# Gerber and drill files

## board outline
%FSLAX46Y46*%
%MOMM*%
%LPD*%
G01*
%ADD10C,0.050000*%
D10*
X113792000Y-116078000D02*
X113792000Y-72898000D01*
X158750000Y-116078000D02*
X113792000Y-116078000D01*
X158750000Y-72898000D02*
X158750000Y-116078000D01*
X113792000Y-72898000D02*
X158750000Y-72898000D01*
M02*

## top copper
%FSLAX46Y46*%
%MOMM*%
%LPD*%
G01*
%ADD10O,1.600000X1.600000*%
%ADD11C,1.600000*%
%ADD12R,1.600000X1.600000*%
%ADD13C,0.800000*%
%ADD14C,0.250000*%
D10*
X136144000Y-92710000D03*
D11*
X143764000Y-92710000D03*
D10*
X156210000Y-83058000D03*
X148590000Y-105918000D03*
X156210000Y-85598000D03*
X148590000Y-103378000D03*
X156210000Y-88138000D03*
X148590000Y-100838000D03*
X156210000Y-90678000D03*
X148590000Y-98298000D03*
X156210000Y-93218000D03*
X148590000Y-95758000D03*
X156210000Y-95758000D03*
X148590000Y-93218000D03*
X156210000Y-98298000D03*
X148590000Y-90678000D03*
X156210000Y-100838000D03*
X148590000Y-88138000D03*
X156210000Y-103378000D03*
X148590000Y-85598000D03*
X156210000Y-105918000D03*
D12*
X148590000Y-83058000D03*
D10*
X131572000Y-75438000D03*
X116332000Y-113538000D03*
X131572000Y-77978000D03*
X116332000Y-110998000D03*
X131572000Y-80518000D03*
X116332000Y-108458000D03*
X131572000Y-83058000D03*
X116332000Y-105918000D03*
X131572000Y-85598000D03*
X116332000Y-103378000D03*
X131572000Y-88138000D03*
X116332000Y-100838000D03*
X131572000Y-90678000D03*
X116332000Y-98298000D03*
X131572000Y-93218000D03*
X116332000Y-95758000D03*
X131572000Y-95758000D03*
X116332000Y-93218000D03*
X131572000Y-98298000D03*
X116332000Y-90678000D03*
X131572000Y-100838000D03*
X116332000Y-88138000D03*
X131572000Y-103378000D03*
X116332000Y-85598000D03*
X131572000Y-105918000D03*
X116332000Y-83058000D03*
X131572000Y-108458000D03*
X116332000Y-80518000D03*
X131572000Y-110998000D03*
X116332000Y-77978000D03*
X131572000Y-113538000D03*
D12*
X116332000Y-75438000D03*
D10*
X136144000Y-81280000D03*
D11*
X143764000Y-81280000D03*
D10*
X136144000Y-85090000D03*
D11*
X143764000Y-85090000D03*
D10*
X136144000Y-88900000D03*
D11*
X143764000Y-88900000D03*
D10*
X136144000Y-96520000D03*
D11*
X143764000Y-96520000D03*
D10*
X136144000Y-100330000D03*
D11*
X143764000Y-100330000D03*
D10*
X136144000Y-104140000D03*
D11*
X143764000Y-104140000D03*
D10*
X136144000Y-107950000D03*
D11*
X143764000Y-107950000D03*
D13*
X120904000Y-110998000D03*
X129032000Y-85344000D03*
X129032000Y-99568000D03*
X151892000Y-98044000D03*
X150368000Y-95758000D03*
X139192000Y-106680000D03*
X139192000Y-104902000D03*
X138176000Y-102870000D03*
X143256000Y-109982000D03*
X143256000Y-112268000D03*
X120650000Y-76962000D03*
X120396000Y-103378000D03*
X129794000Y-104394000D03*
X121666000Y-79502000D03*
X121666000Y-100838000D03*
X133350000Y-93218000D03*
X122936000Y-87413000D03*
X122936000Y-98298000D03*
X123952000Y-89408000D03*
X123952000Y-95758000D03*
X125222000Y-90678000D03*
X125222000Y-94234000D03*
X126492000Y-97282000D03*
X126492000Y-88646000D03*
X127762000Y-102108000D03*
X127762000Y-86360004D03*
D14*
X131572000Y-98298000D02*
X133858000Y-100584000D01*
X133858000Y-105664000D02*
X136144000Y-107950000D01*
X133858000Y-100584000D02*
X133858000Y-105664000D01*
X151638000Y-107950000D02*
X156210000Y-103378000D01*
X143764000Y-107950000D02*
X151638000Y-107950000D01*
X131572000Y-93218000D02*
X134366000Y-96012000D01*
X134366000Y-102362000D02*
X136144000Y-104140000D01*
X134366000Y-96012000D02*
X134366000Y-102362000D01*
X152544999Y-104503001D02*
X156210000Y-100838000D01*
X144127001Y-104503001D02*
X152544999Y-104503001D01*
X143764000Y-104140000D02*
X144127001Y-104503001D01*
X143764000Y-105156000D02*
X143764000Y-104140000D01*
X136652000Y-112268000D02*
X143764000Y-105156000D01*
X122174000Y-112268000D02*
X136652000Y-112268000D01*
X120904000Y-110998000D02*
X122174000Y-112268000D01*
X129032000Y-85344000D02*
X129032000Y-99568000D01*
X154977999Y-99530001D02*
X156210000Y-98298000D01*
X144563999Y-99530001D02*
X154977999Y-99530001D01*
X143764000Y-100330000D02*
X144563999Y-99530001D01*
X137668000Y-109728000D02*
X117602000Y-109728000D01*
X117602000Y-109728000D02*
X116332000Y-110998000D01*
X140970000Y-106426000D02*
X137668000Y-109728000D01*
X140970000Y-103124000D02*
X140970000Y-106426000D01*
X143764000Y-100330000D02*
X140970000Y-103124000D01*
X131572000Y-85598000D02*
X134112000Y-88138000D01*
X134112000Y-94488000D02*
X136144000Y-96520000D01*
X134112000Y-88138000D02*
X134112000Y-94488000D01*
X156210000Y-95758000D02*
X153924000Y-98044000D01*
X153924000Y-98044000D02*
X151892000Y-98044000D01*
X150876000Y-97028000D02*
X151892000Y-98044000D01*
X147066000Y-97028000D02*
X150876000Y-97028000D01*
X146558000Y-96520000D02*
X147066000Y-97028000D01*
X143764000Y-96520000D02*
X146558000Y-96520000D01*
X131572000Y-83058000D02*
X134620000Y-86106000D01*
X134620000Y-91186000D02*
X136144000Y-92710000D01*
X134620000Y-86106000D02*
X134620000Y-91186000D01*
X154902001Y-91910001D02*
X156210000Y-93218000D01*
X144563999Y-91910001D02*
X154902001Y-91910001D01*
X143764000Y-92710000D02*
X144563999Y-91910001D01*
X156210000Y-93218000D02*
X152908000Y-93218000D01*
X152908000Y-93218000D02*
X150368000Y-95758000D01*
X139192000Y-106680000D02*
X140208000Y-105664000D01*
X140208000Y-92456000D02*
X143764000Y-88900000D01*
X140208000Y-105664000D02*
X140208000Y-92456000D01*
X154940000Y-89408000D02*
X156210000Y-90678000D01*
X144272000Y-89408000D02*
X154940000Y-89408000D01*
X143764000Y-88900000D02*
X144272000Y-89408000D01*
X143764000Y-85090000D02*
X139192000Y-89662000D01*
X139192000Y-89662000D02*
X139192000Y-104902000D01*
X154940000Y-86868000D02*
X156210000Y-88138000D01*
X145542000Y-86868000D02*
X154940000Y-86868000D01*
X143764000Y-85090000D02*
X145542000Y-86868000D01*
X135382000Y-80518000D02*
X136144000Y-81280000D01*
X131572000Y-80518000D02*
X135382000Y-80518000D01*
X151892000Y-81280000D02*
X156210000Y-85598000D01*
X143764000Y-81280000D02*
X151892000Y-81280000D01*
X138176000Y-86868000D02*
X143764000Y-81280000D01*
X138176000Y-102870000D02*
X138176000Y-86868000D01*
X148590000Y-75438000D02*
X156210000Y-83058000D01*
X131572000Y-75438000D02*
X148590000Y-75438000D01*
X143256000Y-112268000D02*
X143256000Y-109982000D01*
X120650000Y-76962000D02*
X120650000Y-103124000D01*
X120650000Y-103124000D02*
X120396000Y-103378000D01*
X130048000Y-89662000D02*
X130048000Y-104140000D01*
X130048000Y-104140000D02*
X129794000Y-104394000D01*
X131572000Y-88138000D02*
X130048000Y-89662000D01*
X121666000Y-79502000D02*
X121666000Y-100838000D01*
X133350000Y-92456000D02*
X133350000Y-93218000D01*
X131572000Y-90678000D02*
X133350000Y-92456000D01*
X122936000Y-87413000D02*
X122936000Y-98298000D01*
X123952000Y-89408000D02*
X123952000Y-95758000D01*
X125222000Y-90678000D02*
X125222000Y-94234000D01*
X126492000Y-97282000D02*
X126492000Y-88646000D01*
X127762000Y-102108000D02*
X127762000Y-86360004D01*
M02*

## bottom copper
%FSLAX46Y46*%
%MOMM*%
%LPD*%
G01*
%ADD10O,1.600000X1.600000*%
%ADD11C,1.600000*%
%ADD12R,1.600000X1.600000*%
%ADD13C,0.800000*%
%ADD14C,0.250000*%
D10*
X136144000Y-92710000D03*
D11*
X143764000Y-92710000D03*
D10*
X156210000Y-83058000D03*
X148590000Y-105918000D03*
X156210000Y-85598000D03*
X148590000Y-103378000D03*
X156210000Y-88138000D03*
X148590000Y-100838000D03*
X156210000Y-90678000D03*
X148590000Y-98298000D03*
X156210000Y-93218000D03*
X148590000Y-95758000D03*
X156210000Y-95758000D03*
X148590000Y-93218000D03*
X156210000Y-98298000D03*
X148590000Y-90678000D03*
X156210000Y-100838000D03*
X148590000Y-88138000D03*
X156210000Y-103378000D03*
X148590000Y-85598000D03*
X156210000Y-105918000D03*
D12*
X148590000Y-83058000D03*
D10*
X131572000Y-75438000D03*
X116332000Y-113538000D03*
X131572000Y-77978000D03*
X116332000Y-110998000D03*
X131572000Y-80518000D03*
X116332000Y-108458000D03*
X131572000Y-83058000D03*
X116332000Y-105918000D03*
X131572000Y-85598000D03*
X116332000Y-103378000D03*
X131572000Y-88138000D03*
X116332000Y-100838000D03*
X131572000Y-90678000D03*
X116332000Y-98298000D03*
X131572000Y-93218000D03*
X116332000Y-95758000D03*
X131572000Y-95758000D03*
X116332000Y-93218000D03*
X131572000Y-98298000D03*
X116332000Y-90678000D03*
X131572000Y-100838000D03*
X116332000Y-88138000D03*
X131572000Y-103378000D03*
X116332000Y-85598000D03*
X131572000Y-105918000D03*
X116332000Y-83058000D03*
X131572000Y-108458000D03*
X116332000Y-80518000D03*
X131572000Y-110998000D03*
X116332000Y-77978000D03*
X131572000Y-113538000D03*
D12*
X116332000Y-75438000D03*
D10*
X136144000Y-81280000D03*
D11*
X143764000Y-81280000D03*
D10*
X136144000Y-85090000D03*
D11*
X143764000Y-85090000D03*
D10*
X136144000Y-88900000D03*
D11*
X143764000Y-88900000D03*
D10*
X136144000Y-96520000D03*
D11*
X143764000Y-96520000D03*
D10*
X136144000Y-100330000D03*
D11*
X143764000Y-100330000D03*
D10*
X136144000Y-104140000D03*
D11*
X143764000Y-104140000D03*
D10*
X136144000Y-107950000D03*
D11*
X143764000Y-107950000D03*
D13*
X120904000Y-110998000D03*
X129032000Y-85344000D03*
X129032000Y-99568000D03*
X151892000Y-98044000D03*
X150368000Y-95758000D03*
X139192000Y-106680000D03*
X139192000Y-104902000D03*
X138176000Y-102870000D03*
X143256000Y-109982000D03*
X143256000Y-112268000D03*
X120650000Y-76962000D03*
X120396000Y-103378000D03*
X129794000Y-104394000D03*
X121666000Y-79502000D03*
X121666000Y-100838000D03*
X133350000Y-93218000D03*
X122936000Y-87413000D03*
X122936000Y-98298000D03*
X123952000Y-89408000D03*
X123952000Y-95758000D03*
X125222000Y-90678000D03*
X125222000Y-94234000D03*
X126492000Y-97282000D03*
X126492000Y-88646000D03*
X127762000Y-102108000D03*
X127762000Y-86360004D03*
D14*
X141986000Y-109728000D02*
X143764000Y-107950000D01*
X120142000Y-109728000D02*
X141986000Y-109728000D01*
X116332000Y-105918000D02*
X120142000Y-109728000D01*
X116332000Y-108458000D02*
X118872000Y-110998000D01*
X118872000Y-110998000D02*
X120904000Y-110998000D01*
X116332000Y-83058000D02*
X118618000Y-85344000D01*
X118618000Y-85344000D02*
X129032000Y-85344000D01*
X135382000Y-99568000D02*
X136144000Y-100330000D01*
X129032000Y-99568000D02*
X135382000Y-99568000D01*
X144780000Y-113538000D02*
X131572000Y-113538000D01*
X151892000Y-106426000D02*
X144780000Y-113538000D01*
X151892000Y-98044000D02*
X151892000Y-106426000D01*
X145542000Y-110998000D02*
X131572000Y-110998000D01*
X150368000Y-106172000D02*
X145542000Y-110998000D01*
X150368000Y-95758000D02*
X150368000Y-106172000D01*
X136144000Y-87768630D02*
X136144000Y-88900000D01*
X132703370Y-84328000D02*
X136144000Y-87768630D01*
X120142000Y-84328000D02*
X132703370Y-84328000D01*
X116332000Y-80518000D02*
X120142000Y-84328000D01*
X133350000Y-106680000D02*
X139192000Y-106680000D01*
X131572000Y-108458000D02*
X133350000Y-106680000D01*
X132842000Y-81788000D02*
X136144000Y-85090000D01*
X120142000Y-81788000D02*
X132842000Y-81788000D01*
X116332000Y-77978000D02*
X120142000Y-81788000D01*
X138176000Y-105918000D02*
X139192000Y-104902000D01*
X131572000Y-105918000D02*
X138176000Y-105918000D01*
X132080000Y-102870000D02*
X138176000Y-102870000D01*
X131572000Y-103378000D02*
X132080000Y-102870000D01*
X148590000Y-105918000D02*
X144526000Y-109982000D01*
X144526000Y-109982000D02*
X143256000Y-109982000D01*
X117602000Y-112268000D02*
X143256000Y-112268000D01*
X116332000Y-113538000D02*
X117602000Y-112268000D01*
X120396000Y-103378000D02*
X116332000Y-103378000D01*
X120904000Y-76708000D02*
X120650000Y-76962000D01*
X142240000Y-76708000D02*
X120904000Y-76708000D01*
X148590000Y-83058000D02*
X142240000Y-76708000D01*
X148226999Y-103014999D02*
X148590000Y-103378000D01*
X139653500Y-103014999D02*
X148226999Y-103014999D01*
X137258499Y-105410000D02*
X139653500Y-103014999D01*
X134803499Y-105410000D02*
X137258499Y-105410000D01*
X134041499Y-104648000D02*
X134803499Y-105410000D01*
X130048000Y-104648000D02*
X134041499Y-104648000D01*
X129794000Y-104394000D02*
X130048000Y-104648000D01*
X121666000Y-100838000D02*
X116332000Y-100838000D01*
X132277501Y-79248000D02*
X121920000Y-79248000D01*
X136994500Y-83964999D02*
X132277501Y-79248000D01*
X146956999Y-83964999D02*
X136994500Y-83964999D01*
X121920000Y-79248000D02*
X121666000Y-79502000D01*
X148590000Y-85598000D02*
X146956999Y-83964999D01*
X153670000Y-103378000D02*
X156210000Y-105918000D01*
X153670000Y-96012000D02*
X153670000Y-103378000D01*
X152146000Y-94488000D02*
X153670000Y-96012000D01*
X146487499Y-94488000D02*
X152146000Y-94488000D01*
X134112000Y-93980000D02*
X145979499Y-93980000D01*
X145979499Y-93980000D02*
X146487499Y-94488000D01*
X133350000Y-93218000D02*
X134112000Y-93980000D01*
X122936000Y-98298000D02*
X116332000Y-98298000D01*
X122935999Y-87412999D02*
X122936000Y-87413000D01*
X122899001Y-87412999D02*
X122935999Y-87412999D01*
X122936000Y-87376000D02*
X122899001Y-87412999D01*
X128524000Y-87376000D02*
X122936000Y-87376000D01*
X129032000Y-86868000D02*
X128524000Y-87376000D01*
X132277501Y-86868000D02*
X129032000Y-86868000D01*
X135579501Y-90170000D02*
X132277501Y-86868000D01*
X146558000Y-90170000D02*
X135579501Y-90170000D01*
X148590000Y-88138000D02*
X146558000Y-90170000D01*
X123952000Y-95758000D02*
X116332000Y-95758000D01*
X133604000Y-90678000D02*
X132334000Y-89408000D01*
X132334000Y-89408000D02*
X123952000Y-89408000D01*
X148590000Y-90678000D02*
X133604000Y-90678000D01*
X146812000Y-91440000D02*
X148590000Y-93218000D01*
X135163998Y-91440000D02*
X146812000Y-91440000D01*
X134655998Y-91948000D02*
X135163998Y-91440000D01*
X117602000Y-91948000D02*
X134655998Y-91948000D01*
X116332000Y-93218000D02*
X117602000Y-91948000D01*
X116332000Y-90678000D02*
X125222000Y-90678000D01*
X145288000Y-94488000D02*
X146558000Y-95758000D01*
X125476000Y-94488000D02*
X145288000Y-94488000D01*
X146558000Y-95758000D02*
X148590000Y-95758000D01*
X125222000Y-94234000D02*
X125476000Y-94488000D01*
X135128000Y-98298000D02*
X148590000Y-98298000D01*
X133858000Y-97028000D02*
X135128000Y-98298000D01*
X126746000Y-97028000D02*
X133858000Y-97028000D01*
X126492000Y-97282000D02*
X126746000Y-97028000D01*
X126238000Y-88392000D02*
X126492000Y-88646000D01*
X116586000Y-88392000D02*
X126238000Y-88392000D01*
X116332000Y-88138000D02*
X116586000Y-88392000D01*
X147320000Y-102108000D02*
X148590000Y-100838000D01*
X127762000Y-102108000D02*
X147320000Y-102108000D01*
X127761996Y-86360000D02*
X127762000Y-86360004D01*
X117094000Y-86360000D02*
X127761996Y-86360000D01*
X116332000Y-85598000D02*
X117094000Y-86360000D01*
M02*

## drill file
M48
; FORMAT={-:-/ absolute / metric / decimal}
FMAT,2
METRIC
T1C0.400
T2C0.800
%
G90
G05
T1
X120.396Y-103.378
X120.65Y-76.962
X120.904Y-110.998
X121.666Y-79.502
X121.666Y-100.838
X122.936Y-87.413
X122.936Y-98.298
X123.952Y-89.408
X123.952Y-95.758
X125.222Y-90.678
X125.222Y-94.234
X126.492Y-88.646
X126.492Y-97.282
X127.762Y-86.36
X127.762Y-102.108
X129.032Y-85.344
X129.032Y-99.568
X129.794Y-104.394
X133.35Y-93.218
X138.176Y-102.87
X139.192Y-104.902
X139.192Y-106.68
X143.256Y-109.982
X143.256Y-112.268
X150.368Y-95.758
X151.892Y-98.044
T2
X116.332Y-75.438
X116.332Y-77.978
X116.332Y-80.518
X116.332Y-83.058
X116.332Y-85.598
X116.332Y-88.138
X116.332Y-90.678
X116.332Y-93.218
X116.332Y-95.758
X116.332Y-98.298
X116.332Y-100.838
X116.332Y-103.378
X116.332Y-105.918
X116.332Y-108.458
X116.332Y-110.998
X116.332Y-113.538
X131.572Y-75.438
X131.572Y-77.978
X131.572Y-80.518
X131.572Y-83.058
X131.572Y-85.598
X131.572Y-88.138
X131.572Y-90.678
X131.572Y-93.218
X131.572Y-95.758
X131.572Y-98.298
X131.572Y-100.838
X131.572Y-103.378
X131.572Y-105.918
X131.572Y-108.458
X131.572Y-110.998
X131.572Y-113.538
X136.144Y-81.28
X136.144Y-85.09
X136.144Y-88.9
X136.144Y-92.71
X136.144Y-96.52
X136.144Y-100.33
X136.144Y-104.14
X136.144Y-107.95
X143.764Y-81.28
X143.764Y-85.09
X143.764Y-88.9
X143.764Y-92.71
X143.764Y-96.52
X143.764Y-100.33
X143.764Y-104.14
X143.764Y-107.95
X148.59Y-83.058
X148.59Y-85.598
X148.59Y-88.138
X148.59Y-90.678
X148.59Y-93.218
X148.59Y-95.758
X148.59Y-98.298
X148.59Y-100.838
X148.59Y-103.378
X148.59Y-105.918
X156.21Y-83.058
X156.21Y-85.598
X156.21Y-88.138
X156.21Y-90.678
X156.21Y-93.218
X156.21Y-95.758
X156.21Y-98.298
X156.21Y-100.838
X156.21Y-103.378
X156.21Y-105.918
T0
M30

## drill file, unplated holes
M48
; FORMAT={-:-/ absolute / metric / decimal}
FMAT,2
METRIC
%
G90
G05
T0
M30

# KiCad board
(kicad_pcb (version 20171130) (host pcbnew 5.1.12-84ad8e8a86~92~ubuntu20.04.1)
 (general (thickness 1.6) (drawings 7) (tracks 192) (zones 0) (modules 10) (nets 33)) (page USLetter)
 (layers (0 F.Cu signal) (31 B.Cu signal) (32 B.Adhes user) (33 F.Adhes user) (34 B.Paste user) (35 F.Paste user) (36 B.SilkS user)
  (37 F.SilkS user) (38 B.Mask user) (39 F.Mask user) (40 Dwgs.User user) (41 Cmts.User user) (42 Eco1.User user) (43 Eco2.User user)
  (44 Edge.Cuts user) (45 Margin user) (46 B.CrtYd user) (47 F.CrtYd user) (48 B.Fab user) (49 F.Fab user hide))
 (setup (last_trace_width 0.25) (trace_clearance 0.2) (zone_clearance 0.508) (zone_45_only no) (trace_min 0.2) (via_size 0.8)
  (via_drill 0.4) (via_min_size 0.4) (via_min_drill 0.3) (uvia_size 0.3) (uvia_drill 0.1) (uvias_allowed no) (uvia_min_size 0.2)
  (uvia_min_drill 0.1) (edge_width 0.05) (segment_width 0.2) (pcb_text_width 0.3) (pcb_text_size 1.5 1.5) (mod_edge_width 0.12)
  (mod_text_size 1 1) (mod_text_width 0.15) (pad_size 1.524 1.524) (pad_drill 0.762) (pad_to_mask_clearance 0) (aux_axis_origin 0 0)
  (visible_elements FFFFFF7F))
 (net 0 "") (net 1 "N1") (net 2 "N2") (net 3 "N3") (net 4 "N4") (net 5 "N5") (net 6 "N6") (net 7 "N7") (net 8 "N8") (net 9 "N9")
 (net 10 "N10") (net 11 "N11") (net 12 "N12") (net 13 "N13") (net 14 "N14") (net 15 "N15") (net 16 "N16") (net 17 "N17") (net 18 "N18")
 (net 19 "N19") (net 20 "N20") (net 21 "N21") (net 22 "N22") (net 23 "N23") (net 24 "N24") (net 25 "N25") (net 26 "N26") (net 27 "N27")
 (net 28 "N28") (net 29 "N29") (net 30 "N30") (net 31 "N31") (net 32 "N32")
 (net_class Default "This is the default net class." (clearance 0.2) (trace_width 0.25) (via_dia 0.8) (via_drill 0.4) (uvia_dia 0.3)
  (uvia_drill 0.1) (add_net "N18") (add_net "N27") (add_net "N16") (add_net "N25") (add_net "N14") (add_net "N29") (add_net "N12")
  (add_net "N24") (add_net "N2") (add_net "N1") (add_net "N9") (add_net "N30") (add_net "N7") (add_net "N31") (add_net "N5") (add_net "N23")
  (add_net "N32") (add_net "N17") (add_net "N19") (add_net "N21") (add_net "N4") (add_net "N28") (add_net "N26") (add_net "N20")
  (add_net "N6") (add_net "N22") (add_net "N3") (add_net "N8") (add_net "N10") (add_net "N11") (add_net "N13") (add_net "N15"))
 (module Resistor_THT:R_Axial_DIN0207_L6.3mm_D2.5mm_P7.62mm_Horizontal (layer F.Cu) (at 143.764 92.71 180)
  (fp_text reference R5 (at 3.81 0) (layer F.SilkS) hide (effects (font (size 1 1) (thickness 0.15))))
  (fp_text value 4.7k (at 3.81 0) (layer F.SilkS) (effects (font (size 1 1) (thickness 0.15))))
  (pad 2 thru_hole oval (at 7.62 0 180) (size 1.6 1.6) (drill 0.8) (layers *.Cu *.Mask) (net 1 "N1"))
  (pad 1 thru_hole circle (at 0 0 180) (size 1.6 1.6) (drill 0.8) (layers *.Cu *.Mask) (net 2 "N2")))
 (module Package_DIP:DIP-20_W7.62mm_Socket (layer F.Cu) (at 148.59 83.058)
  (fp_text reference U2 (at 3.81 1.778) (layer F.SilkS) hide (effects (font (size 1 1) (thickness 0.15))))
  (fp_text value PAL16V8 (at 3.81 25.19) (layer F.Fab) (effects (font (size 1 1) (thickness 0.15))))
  (pad 20 thru_hole oval (at 7.62 0) (size 1.6 1.6) (drill 0.8) (layers *.Cu *.Mask) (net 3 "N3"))
  (pad 10 thru_hole oval (at 0 22.86) (size 1.6 1.6) (drill 0.8) (layers *.Cu *.Mask) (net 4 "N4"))
  (pad 19 thru_hole oval (at 7.62 2.54) (size 1.6 1.6) (drill 0.8) (layers *.Cu *.Mask) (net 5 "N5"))
  (pad 9 thru_hole oval (at 0 20.32) (size 1.6 1.6) (drill 0.8) (layers *.Cu *.Mask) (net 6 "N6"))
  (pad 18 thru_hole oval (at 7.62 5.08) (size 1.6 1.6) (drill 0.8) (layers *.Cu *.Mask) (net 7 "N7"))
  (pad 8 thru_hole oval (at 0 17.78) (size 1.6 1.6) (drill 0.8) (layers *.Cu *.Mask) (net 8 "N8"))
  (pad 17 thru_hole oval (at 7.62 7.62) (size 1.6 1.6) (drill 0.8) (layers *.Cu *.Mask) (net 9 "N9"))
  (pad 7 thru_hole oval (at 0 15.24) (size 1.6 1.6) (drill 0.8) (layers *.Cu *.Mask) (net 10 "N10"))
  (pad 16 thru_hole oval (at 7.62 10.16) (size 1.6 1.6) (drill 0.8) (layers *.Cu *.Mask) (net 2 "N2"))
  (pad 6 thru_hole oval (at 0 12.7) (size 1.6 1.6) (drill 0.8) (layers *.Cu *.Mask) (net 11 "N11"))
  (pad 15 thru_hole oval (at 7.62 12.7) (size 1.6 1.6) (drill 0.8) (layers *.Cu *.Mask) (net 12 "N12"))
  (pad 5 thru_hole oval (at 0 10.16) (size 1.6 1.6) (drill 0.8) (layers *.Cu *.Mask) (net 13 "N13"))
  (pad 14 thru_hole oval (at 7.62 15.24) (size 1.6 1.6) (drill 0.8) (layers *.Cu *.Mask) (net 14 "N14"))
  (pad 4 thru_hole oval (at 0 7.62) (size 1.6 1.6) (drill 0.8) (layers *.Cu *.Mask) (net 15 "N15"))
  (pad 13 thru_hole oval (at 7.62 17.78) (size 1.6 1.6) (drill 0.8) (layers *.Cu *.Mask) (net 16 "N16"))
  (pad 3 thru_hole oval (at 0 5.08) (size 1.6 1.6) (drill 0.8) (layers *.Cu *.Mask) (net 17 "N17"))
  (pad 12 thru_hole oval (at 7.62 20.32) (size 1.6 1.6) (drill 0.8) (layers *.Cu *.Mask) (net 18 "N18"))
  (pad 2 thru_hole oval (at 0 2.54) (size 1.6 1.6) (drill 0.8) (layers *.Cu *.Mask) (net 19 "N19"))
  (pad 11 thru_hole oval (at 7.62 22.86) (size 1.6 1.6) (drill 0.8) (layers *.Cu *.Mask) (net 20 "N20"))
  (pad 1 thru_hole rect (at 0 0) (size 1.6 1.6) (drill 0.8) (layers *.Cu *.Mask) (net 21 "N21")))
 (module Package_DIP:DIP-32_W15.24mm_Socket (layer F.Cu) (at 116.332 75.438)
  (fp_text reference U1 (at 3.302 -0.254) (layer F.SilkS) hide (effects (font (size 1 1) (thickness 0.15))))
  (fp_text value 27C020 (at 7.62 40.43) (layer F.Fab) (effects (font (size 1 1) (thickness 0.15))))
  (pad 32 thru_hole oval (at 15.24 0) (size 1.6 1.6) (drill 0.8) (layers *.Cu *.Mask) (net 3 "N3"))
  (pad 16 thru_hole oval (at 0 38.1) (size 1.6 1.6) (drill 0.8) (layers *.Cu *.Mask) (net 4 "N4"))
  (pad 31 thru_hole oval (at 15.24 2.54) (size 1.6 1.6) (drill 0.8) (layers *.Cu *.Mask) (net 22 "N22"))
  (pad 15 thru_hole oval (at 0 35.56) (size 1.6 1.6) (drill 0.8) (layers *.Cu *.Mask) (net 14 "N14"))
  (pad 30 thru_hole oval (at 15.24 5.08) (size 1.6 1.6) (drill 0.8) (layers *.Cu *.Mask) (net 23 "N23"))
  (pad 14 thru_hole oval (at 0 33.02) (size 1.6 1.6) (drill 0.8) (layers *.Cu *.Mask) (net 16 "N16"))
  (pad 29 thru_hole oval (at 15.24 7.62) (size 1.6 1.6) (drill 0.8) (layers *.Cu *.Mask) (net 1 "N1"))
  (pad 13 thru_hole oval (at 0 30.48) (size 1.6 1.6) (drill 0.8) (layers *.Cu *.Mask) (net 18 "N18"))
  (pad 28 thru_hole oval (at 15.24 10.16) (size 1.6 1.6) (drill 0.8) (layers *.Cu *.Mask) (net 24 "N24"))
  (pad 12 thru_hole oval (at 0 27.94) (size 1.6 1.6) (drill 0.8) (layers *.Cu *.Mask) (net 21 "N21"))
  (pad 27 thru_hole oval (at 15.24 12.7) (size 1.6 1.6) (drill 0.8) (layers *.Cu *.Mask) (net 6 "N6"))
  (pad 11 thru_hole oval (at 0 25.4) (size 1.6 1.6) (drill 0.8) (layers *.Cu *.Mask) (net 19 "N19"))
  (pad 26 thru_hole oval (at 15.24 15.24) (size 1.6 1.6) (drill 0.8) (layers *.Cu *.Mask) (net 20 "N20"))
  (pad 10 thru_hole oval (at 0 22.86) (size 1.6 1.6) (drill 0.8) (layers *.Cu *.Mask) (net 17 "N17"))
  (pad 25 thru_hole oval (at 15.24 17.78) (size 1.6 1.6) (drill 0.8) (layers *.Cu *.Mask) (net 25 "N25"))
  (pad 9 thru_hole oval (at 0 20.32) (size 1.6 1.6) (drill 0.8) (layers *.Cu *.Mask) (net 15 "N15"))
  (pad 24 thru_hole oval (at 15.24 20.32) (size 1.6 1.6) (drill 0.8) (layers *.Cu *.Mask) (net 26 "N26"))
  (pad 8 thru_hole oval (at 0 17.78) (size 1.6 1.6) (drill 0.8) (layers *.Cu *.Mask) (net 13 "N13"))
  (pad 23 thru_hole oval (at 15.24 22.86) (size 1.6 1.6) (drill 0.8) (layers *.Cu *.Mask) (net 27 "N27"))
  (pad 7 thru_hole oval (at 0 15.24) (size 1.6 1.6) (drill 0.8) (layers *.Cu *.Mask) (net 11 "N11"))
  (pad 22 thru_hole oval (at 15.24 25.4) (size 1.6 1.6) (drill 0.8) (layers *.Cu *.Mask) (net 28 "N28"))
  (pad 6 thru_hole oval (at 0 12.7) (size 1.6 1.6) (drill 0.8) (layers *.Cu *.Mask) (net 10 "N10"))
  (pad 21 thru_hole oval (at 15.24 27.94) (size 1.6 1.6) (drill 0.8) (layers *.Cu *.Mask) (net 5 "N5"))
  (pad 5 thru_hole oval (at 0 10.16) (size 1.6 1.6) (drill 0.8) (layers *.Cu *.Mask) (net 8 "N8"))
  (pad 20 thru_hole oval (at 15.24 30.48) (size 1.6 1.6) (drill 0.8) (layers *.Cu *.Mask) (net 7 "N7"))
  (pad 4 thru_hole oval (at 0 7.62) (size 1.6 1.6) (drill 0.8) (layers *.Cu *.Mask) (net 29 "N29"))
  (pad 19 thru_hole oval (at 15.24 33.02) (size 1.6 1.6) (drill 0.8) (layers *.Cu *.Mask) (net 9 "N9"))
  (pad 3 thru_hole oval (at 0 5.08) (size 1.6 1.6) (drill 0.8) (layers *.Cu *.Mask) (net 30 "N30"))
  (pad 18 thru_hole oval (at 15.24 35.56) (size 1.6 1.6) (drill 0.8) (layers *.Cu *.Mask) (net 2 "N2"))
  (pad 2 thru_hole oval (at 0 2.54) (size 1.6 1.6) (drill 0.8) (layers *.Cu *.Mask) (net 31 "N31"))
  (pad 17 thru_hole oval (at 15.24 38.1) (size 1.6 1.6) (drill 0.8) (layers *.Cu *.Mask) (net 12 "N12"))
  (pad 1 thru_hole rect (at 0 0) (size 1.6 1.6) (drill 0.8) (layers *.Cu *.Mask) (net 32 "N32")))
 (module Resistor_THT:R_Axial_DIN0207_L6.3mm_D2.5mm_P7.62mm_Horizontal (layer F.Cu) (at 143.764 81.28 180)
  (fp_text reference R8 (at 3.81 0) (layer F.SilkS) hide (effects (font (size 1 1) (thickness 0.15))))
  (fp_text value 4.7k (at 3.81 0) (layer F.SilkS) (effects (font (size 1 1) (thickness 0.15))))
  (pad 2 thru_hole oval (at 7.62 0 180) (size 1.6 1.6) (drill 0.8) (layers *.Cu *.Mask) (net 23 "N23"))
  (pad 1 thru_hole circle (at 0 0 180) (size 1.6 1.6) (drill 0.8) (layers *.Cu *.Mask) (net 5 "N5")))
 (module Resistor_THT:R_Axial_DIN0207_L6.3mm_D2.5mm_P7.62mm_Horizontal (layer F.Cu) (at 143.764 85.09 180)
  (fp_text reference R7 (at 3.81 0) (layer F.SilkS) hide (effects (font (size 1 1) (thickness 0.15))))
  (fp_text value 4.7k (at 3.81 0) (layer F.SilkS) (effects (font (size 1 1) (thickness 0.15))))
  (pad 2 thru_hole oval (at 7.62 0 180) (size 1.6 1.6) (drill 0.8) (layers *.Cu *.Mask) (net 31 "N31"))
  (pad 1 thru_hole circle (at 0 0 180) (size 1.6 1.6) (drill 0.8) (layers *.Cu *.Mask) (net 7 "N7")))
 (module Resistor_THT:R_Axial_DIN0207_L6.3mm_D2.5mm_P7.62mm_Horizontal (layer F.Cu) (at 143.764 88.9 180)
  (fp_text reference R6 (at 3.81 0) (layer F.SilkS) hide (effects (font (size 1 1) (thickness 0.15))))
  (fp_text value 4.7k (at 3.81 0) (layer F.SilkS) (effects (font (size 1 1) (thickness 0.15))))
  (pad 2 thru_hole oval (at 7.62 0 180) (size 1.6 1.6) (drill 0.8) (layers *.Cu *.Mask) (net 30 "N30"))
  (pad 1 thru_hole circle (at 0 0 180) (size 1.6 1.6) (drill 0.8) (layers *.Cu *.Mask) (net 9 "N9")))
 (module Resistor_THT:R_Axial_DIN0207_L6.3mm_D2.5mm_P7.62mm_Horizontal (layer F.Cu) (at 143.764 96.52 180)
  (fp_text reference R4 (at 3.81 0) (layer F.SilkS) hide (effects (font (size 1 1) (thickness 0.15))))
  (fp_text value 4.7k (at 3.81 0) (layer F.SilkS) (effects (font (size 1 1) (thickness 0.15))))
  (pad 2 thru_hole oval (at 7.62 0 180) (size 1.6 1.6) (drill 0.8) (layers *.Cu *.Mask) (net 24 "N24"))
  (pad 1 thru_hole circle (at 0 0 180) (size 1.6 1.6) (drill 0.8) (layers *.Cu *.Mask) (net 12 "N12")))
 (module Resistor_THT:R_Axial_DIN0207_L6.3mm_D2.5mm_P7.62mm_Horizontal (layer F.Cu) (at 143.764 100.33 180)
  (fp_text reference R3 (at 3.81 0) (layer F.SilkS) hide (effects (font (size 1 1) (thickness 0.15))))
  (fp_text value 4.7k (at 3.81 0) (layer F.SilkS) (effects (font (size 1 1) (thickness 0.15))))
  (pad 2 thru_hole oval (at 7.62 0 180) (size 1.6 1.6) (drill 0.8) (layers *.Cu *.Mask) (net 29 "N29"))
  (pad 1 thru_hole circle (at 0 0 180) (size 1.6 1.6) (drill 0.8) (layers *.Cu *.Mask) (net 14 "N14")))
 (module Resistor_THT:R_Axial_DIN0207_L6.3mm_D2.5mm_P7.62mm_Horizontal (layer F.Cu) (at 143.764 104.14 180)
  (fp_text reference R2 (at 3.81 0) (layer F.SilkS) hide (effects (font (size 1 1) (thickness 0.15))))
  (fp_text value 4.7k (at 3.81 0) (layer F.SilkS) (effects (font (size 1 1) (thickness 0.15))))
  (pad 2 thru_hole oval (at 7.62 0 180) (size 1.6 1.6) (drill 0.8) (layers *.Cu *.Mask) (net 25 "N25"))
  (pad 1 thru_hole circle (at 0 0 180) (size 1.6 1.6) (drill 0.8) (layers *.Cu *.Mask) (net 16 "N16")))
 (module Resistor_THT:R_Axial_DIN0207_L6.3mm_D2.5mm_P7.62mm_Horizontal (layer F.Cu) (at 143.764 107.95 180)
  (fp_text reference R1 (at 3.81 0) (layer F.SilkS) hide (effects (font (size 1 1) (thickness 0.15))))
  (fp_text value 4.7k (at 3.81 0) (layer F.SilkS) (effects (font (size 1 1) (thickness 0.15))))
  (pad 2 thru_hole oval (at 7.62 0 180) (size 1.6 1.6) (drill 0.8) (layers *.Cu *.Mask) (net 27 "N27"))
  (pad 1 thru_hole circle (at 0 0 180) (size 1.6 1.6) (drill 0.8) (layers *.Cu *.Mask) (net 18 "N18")))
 (gr_line (start 113.792 116.078) (end 113.792 72.898) (layer Edge.Cuts) (width 0.05))
 (gr_line (start 158.75 116.078) (end 113.792 116.078) (layer Edge.Cuts) (width 0.05))
 (gr_line (start 158.75 72.898) (end 158.75 116.078) (layer Edge.Cuts) (width 0.05))
 (gr_line (start 113.792 72.898) (end 158.75 72.898) (layer Edge.Cuts) (width 0.05))
 (segment (start 131.572 98.298) (end 133.858 100.584) (width 0.25) (layer F.Cu) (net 27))
 (segment (start 133.858 105.664) (end 136.144 107.95) (width 0.25) (layer F.Cu) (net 27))
 (segment (start 133.858 100.584) (end 133.858 105.664) (width 0.25) (layer F.Cu) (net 27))
 (segment (start 151.638 107.95) (end 156.21 103.378) (width 0.25) (layer F.Cu) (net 18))
 (segment (start 143.764 107.95) (end 151.638 107.95) (width 0.25) (layer F.Cu) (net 18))
 (segment (start 141.986 109.728) (end 143.764 107.95) (width 0.25) (layer B.Cu) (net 18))
 (segment (start 120.142 109.728) (end 141.986 109.728) (width 0.25) (layer B.Cu) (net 18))
 (segment (start 116.332 105.918) (end 120.142 109.728) (width 0.25) (layer B.Cu) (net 18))
 (segment (start 131.572 93.218) (end 134.366 96.012) (width 0.25) (layer F.Cu) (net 25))
 (segment (start 134.366 102.362) (end 136.144 104.14) (width 0.25) (layer F.Cu) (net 25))
 (segment (start 134.366 96.012) (end 134.366 102.362) (width 0.25) (layer F.Cu) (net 25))
 (segment (start 152.544999 104.503001) (end 156.21 100.838) (width 0.25) (layer F.Cu) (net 16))
 (segment (start 144.127001 104.503001) (end 152.544999 104.503001) (width 0.25) (layer F.Cu) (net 16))
 (segment (start 143.764 104.14) (end 144.127001 104.503001) (width 0.25) (layer F.Cu) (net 16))
 (segment (start 116.332 108.458) (end 118.872 110.998) (width 0.25) (layer B.Cu) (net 16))
 (via (at 120.904 110.998) (size 0.8) (drill 0.4) (layers F.Cu B.Cu) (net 16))
 (segment (start 118.872 110.998) (end 120.904 110.998) (width 0.25) (layer B.Cu) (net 16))
 (segment (start 143.764 105.156) (end 143.764 104.14) (width 0.25) (layer F.Cu) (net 16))
 (segment (start 136.652 112.268) (end 143.764 105.156) (width 0.25) (layer F.Cu) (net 16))
 (segment (start 122.174 112.268) (end 136.652 112.268) (width 0.25) (layer F.Cu) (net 16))
 (segment (start 120.904 110.998) (end 122.174 112.268) (width 0.25) (layer F.Cu) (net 16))
 (segment (start 116.332 83.058) (end 118.618 85.344) (width 0.25) (layer B.Cu) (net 29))
 (segment (start 118.618 85.344) (end 129.032 85.344) (width 0.25) (layer B.Cu) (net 29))
 (via (at 129.032 85.344) (size 0.8) (drill 0.4) (layers F.Cu B.Cu) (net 29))
 (segment (start 129.032 85.344) (end 129.032 99.568) (width 0.25) (layer F.Cu) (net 29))
 (via (at 129.032 99.568) (size 0.8) (drill 0.4) (layers F.Cu B.Cu) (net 29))
 (segment (start 135.382 99.568) (end 136.144 100.33) (width 0.25) (layer B.Cu) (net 29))
 (segment (start 129.032 99.568) (end 135.382 99.568) (width 0.25) (layer B.Cu) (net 29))
 (segment (start 154.977999 99.530001) (end 156.21 98.298) (width 0.25) (layer F.Cu) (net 14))
 (segment (start 144.563999 99.530001) (end 154.977999 99.530001) (width 0.25) (layer F.Cu) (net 14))
 (segment (start 143.764 100.33) (end 144.563999 99.530001) (width 0.25) (layer F.Cu) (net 14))
 (segment (start 137.668 109.728) (end 117.602 109.728) (width 0.25) (layer F.Cu) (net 14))
 (segment (start 117.602 109.728) (end 116.332 110.998) (width 0.25) (layer F.Cu) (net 14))
 (segment (start 140.97 106.426) (end 137.668 109.728) (width 0.25) (layer F.Cu) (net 14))
 (segment (start 140.97 103.124) (end 140.97 106.426) (width 0.25) (layer F.Cu) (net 14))
 (segment (start 143.764 100.33) (end 140.97 103.124) (width 0.25) (layer F.Cu) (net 14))
 (segment (start 131.572 85.598) (end 134.112 88.138) (width 0.25) (layer F.Cu) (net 24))
 (segment (start 134.112 94.488) (end 136.144 96.52) (width 0.25) (layer F.Cu) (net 24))
 (segment (start 134.112 88.138) (end 134.112 94.488) (width 0.25) (layer F.Cu) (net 24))
 (segment (start 156.21 95.758) (end 153.924 98.044) (width 0.25) (layer F.Cu) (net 12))
 (via (at 151.892 98.044) (size 0.8) (drill 0.4) (layers F.Cu B.Cu) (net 12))
 (segment (start 153.924 98.044) (end 151.892 98.044) (width 0.25) (layer F.Cu) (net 12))
 (segment (start 144.78 113.538) (end 131.572 113.538) (width 0.25) (layer B.Cu) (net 12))
 (segment (start 151.892 106.426) (end 144.78 113.538) (width 0.25) (layer B.Cu) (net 12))
 (segment (start 151.892 98.044) (end 151.892 106.426) (width 0.25) (layer B.Cu) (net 12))
 (segment (start 150.876 97.028) (end 151.892 98.044) (width 0.25) (layer F.Cu) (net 12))
 (segment (start 147.066 97.028) (end 150.876 97.028) (width 0.25) (layer F.Cu) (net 12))
 (segment (start 146.558 96.52) (end 147.066 97.028) (width 0.25) (layer F.Cu) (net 12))
 (segment (start 143.764 96.52) (end 146.558 96.52) (width 0.25) (layer F.Cu) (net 12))
 (segment (start 131.572 83.058) (end 134.62 86.106) (width 0.25) (layer F.Cu) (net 1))
 (segment (start 134.62 91.186) (end 136.144 92.71) (width 0.25) (layer F.Cu) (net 1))
 (segment (start 134.62 86.106) (end 134.62 91.186) (width 0.25) (layer F.Cu) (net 1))
 (segment (start 154.902001 91.910001) (end 156.21 93.218) (width 0.25) (layer F.Cu) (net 2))
 (segment (start 144.563999 91.910001) (end 154.902001 91.910001) (width 0.25) (layer F.Cu) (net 2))
 (segment (start 143.764 92.71) (end 144.563999 91.910001) (width 0.25) (layer F.Cu) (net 2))
 (segment (start 156.21 93.218) (end 152.908 93.218) (width 0.25) (layer F.Cu) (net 2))
 (via (at 150.368 95.758) (size 0.8) (drill 0.4) (layers F.Cu B.Cu) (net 2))
 (segment (start 152.908 93.218) (end 150.368 95.758) (width 0.25) (layer F.Cu) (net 2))
 (segment (start 145.542 110.998) (end 131.572 110.998) (width 0.25) (layer B.Cu) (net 2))
 (segment (start 150.368 106.172) (end 145.542 110.998) (width 0.25) (layer B.Cu) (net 2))
 (segment (start 150.368 95.758) (end 150.368 106.172) (width 0.25) (layer B.Cu) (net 2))
 (segment (start 136.144 87.76863) (end 136.144 88.9) (width 0.25) (layer B.Cu) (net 30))
 (segment (start 132.70337 84.328) (end 136.144 87.76863) (width 0.25) (layer B.Cu) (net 30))
 (segment (start 120.142 84.328) (end 132.70337 84.328) (width 0.25) (layer B.Cu) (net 30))
 (segment (start 116.332 80.518) (end 120.142 84.328) (width 0.25) (layer B.Cu) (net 30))
 (via (at 139.192 106.68) (size 0.8) (drill 0.4) (layers F.Cu B.Cu) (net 9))
 (segment (start 139.192 106.68) (end 140.208 105.664) (width 0.25) (layer F.Cu) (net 9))
 (segment (start 140.208 92.456) (end 143.764 88.9) (width 0.25) (layer F.Cu) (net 9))
 (segment (start 140.208 105.664) (end 140.208 92.456) (width 0.25) (layer F.Cu) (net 9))
 (segment (start 133.35 106.68) (end 139.192 106.68) (width 0.25) (layer B.Cu) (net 9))
 (segment (start 131.572 108.458) (end 133.35 106.68) (width 0.25) (layer B.Cu) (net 9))
 (segment (start 154.94 89.408) (end 156.21 90.678) (width 0.25) (layer F.Cu) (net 9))
 (segment (start 144.272 89.408) (end 154.94 89.408) (width 0.25) (layer F.Cu) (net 9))
 (segment (start 143.764 88.9) (end 144.272 89.408) (width 0.25) (layer F.Cu) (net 9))
 (segment (start 132.842 81.788) (end 136.144 85.09) (width 0.25) (layer B.Cu) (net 31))
 (segment (start 120.142 81.788) (end 132.842 81.788) (width 0.25) (layer B.Cu) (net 31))
 (segment (start 116.332 77.978) (end 120.142 81.788) (width 0.25) (layer B.Cu) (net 31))
 (via (at 139.192 104.902) (size 0.8) (drill 0.4) (layers F.Cu B.Cu) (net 7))
 (segment (start 143.764 85.09) (end 139.192 89.662) (width 0.25) (layer F.Cu) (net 7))
 (segment (start 139.192 89.662) (end 139.192 104.902) (width 0.25) (layer F.Cu) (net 7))
 (segment (start 154.94 86.868) (end 156.21 88.138) (width 0.25) (layer F.Cu) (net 7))
 (segment (start 145.542 86.868) (end 154.94 86.868) (width 0.25) (layer F.Cu) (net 7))
 (segment (start 143.764 85.09) (end 145.542 86.868) (width 0.25) (layer F.Cu) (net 7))
 (segment (start 138.176 105.918) (end 139.192 104.902) (width 0.25) (layer B.Cu) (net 7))
 (segment (start 131.572 105.918) (end 138.176 105.918) (width 0.25) (layer B.Cu) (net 7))
 (segment (start 135.382 80.518) (end 136.144 81.28) (width 0.25) (layer F.Cu) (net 23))
 (segment (start 131.572 80.518) (end 135.382 80.518) (width 0.25) (layer F.Cu) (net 23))
 (segment (start 151.892 81.28) (end 156.21 85.598) (width 0.25) (layer F.Cu) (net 5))
 (segment (start 143.764 81.28) (end 151.892 81.28) (width 0.25) (layer F.Cu) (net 5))
 (via (at 138.176 102.87) (size 0.8) (drill 0.4) (layers F.Cu B.Cu) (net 5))
 (segment (start 132.08 102.87) (end 138.176 102.87) (width 0.25) (layer B.Cu) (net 5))
 (segment (start 131.572 103.378) (end 132.08 102.87) (width 0.25) (layer B.Cu) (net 5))
 (segment (start 138.176 86.868) (end 143.764 81.28) (width 0.25) (layer F.Cu) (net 5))
 (segment (start 138.176 102.87) (end 138.176 86.868) (width 0.25) (layer F.Cu) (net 5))
 (segment (start 148.59 75.438) (end 156.21 83.058) (width 0.25) (layer F.Cu) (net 3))
 (segment (start 131.572 75.438) (end 148.59 75.438) (width 0.25) (layer F.Cu) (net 3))
 (segment (start 148.59 105.918) (end 144.526 109.982) (width 0.25) (layer B.Cu) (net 4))
 (via (at 143.256 109.982) (size 0.8) (drill 0.4) (layers F.Cu B.Cu) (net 4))
 (segment (start 144.526 109.982) (end 143.256 109.982) (width 0.25) (layer B.Cu) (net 4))
 (segment (start 117.602 112.268) (end 143.256 112.268) (width 0.25) (layer B.Cu) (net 4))
 (via (at 143.256 112.268) (size 0.8) (drill 0.4) (layers F.Cu B.Cu) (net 4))
 (segment (start 116.332 113.538) (end 117.602 112.268) (width 0.25) (layer B.Cu) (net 4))
 (segment (start 143.256 112.268) (end 143.256 109.982) (width 0.25) (layer F.Cu) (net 4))
 (via (at 120.65 76.962) (size 0.8) (drill 0.4) (layers F.Cu B.Cu) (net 21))
 (segment (start 120.65 76.962) (end 120.65 103.124) (width 0.25) (layer F.Cu) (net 21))
 (via (at 120.396 103.378) (size 0.8) (drill 0.4) (layers F.Cu B.Cu) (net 21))
 (segment (start 120.65 103.124) (end 120.396 103.378) (width 0.25) (layer F.Cu) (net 21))
 (segment (start 120.396 103.378) (end 116.332 103.378) (width 0.25) (layer B.Cu) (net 21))
 (segment (start 120.904 76.708) (end 120.65 76.962) (width 0.25) (layer B.Cu) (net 21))
 (segment (start 142.24 76.708) (end 120.904 76.708) (width 0.25) (layer B.Cu) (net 21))
 (segment (start 148.59 83.058) (end 142.24 76.708) (width 0.25) (layer B.Cu) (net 21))
 (via (at 129.794 104.394) (size 0.8) (drill 0.4) (layers F.Cu B.Cu) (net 6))
 (segment (start 130.048 89.662) (end 130.048 104.14) (width 0.25) (layer F.Cu) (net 6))
 (segment (start 130.048 104.14) (end 129.794 104.394) (width 0.25) (layer F.Cu) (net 6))
 (segment (start 131.572 88.138) (end 130.048 89.662) (width 0.25) (layer F.Cu) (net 6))
 (segment (start 148.226999 103.014999) (end 148.59 103.378) (width 0.25) (layer B.Cu) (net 6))
 (segment (start 139.6535 103.014999) (end 148.226999 103.014999) (width 0.25) (layer B.Cu) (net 6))
 (segment (start 137.258499 105.41) (end 139.6535 103.014999) (width 0.25) (layer B.Cu) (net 6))
 (segment (start 134.803499 105.41) (end 137.258499 105.41) (width 0.25) (layer B.Cu) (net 6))
 (segment (start 134.041499 104.648) (end 134.803499 105.41) (width 0.25) (layer B.Cu) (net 6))
 (segment (start 130.048 104.648) (end 134.041499 104.648) (width 0.25) (layer B.Cu) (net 6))
 (segment (start 129.794 104.394) (end 130.048 104.648) (width 0.25) (layer B.Cu) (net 6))
 (via (at 121.666 79.502) (size 0.8) (drill 0.4) (layers F.Cu B.Cu) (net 19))
 (segment (start 121.666 79.502) (end 121.666 100.838) (width 0.25) (layer F.Cu) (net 19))
 (via (at 121.666 100.838) (size 0.8) (drill 0.4) (layers F.Cu B.Cu) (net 19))
 (segment (start 121.666 100.838) (end 116.332 100.838) (width 0.25) (layer B.Cu) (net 19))
 (segment (start 132.277501 79.248) (end 121.92 79.248) (width 0.25) (layer B.Cu) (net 19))
 (segment (start 136.9945 83.964999) (end 132.277501 79.248) (width 0.25) (layer B.Cu) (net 19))
 (segment (start 146.956999 83.964999) (end 136.9945 83.964999) (width 0.25) (layer B.Cu) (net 19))
 (segment (start 121.92 79.248) (end 121.666 79.502) (width 0.25) (layer B.Cu) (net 19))
 (segment (start 148.59 85.598) (end 146.956999 83.964999) (width 0.25) (layer B.Cu) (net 19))
 (via (at 133.35 93.218) (size 0.8) (drill 0.4) (layers F.Cu B.Cu) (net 20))
 (segment (start 133.35 92.456) (end 133.35 93.218) (width 0.25) (layer F.Cu) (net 20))
 (segment (start 131.572 90.678) (end 133.35 92.456) (width 0.25) (layer F.Cu) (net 20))
 (segment (start 153.67 103.378) (end 156.21 105.918) (width 0.25) (layer B.Cu) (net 20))
 (segment (start 153.67 96.012) (end 153.67 103.378) (width 0.25) (layer B.Cu) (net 20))
 (segment (start 152.146 94.488) (end 153.67 96.012) (width 0.25) (layer B.Cu) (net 20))
 (segment (start 146.487499 94.488) (end 152.146 94.488) (width 0.25) (layer B.Cu) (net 20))
 (segment (start 134.112 93.98) (end 145.979499 93.98) (width 0.25) (layer B.Cu) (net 20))
 (segment (start 145.979499 93.98) (end 146.487499 94.488) (width 0.25) (layer B.Cu) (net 20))
 (segment (start 133.35 93.218) (end 134.112 93.98) (width 0.25) (layer B.Cu) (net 20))
 (via (at 122.936 87.413) (size 0.8) (drill 0.4) (layers F.Cu B.Cu) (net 17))
 (via (at 122.936 98.298) (size 0.8) (drill 0.4) (layers F.Cu B.Cu) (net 17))
 (segment (start 122.936 87.413) (end 122.936 98.298) (width 0.25) (layer F.Cu) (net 17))
 (segment (start 122.936 98.298) (end 116.332 98.298) (width 0.25) (layer B.Cu) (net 17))
 (segment (start 122.935999 87.412999) (end 122.936 87.413) (width 0.25) (layer B.Cu) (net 17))
 (segment (start 122.899001 87.412999) (end 122.935999 87.412999) (width 0.25) (layer B.Cu) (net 17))
 (segment (start 122.936 87.376) (end 122.899001 87.412999) (width 0.25) (layer B.Cu) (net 17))
 (segment (start 128.524 87.376) (end 122.936 87.376) (width 0.25) (layer B.Cu) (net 17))
 (segment (start 129.032 86.868) (end 128.524 87.376) (width 0.25) (layer B.Cu) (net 17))
 (segment (start 132.277501 86.868) (end 129.032 86.868) (width 0.25) (layer B.Cu) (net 17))
 (segment (start 135.579501 90.17) (end 132.277501 86.868) (width 0.25) (layer B.Cu) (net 17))
 (segment (start 146.558 90.17) (end 135.579501 90.17) (width 0.25) (layer B.Cu) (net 17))
 (segment (start 148.59 88.138) (end 146.558 90.17) (width 0.25) (layer B.Cu) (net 17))
 (via (at 123.952 89.408) (size 0.8) (drill 0.4) (layers F.Cu B.Cu) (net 15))
 (segment (start 123.952 89.408) (end 123.952 95.758) (width 0.25) (layer F.Cu) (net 15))
 (via (at 123.952 95.758) (size 0.8) (drill 0.4) (layers F.Cu B.Cu) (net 15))
 (segment (start 123.952 95.758) (end 116.332 95.758) (width 0.25) (layer B.Cu) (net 15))
 (segment (start 133.604 90.678) (end 132.334 89.408) (width 0.25) (layer B.Cu) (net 15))
 (segment (start 132.334 89.408) (end 123.952 89.408) (width 0.25) (layer B.Cu) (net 15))
 (segment (start 148.59 90.678) (end 133.604 90.678) (width 0.25) (layer B.Cu) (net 15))
 (segment (start 146.812 91.44) (end 148.59 93.218) (width 0.25) (layer B.Cu) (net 13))
 (segment (start 135.163998 91.44) (end 146.812 91.44) (width 0.25) (layer B.Cu) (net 13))
 (segment (start 134.655998 91.948) (end 135.163998 91.44) (width 0.25) (layer B.Cu) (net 13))
 (segment (start 117.602 91.948) (end 134.655998 91.948) (width 0.25) (layer B.Cu) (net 13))
 (segment (start 116.332 93.218) (end 117.602 91.948) (width 0.25) (layer B.Cu) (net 13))
 (segment (start 116.332 90.678) (end 125.222 90.678) (width 0.25) (layer B.Cu) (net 11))
 (via (at 125.222 90.678) (size 0.8) (drill 0.4) (layers F.Cu B.Cu) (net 11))
 (via (at 125.222 94.234) (size 0.8) (drill 0.4) (layers F.Cu B.Cu) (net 11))
 (segment (start 125.222 90.678) (end 125.222 94.234) (width 0.25) (layer F.Cu) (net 11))
 (segment (start 145.288 94.488) (end 146.558 95.758) (width 0.25) (layer B.Cu) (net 11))
 (segment (start 125.476 94.488) (end 145.288 94.488) (width 0.25) (layer B.Cu) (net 11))
 (segment (start 146.558 95.758) (end 148.59 95.758) (width 0.25) (layer B.Cu) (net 11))
 (segment (start 125.222 94.234) (end 125.476 94.488) (width 0.25) (layer B.Cu) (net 11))
 (via (at 126.492 97.282) (size 0.8) (drill 0.4) (layers F.Cu B.Cu) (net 10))
 (segment (start 135.128 98.298) (end 148.59 98.298) (width 0.25) (layer B.Cu) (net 10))
 (segment (start 133.858 97.028) (end 135.128 98.298) (width 0.25) (layer B.Cu) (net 10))
 (segment (start 126.746 97.028) (end 133.858 97.028) (width 0.25) (layer B.Cu) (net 10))
 (segment (start 126.492 97.282) (end 126.746 97.028) (width 0.25) (layer B.Cu) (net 10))
 (via (at 126.492 88.646) (size 0.8) (drill 0.4) (layers F.Cu B.Cu) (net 10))
 (segment (start 126.492 97.282) (end 126.492 88.646) (width 0.25) (layer F.Cu) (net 10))
 (segment (start 126.238 88.392) (end 126.492 88.646) (width 0.25) (layer B.Cu) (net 10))
 (segment (start 116.586 88.392) (end 126.238 88.392) (width 0.25) (layer B.Cu) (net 10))
 (segment (start 116.332 88.138) (end 116.586 88.392) (width 0.25) (layer B.Cu) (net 10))
 (via (at 127.762 102.108) (size 0.8) (drill 0.4) (layers F.Cu B.Cu) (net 8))
 (segment (start 147.32 102.108) (end 148.59 100.838) (width 0.25) (layer B.Cu) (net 8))
 (segment (start 127.762 102.108) (end 147.32 102.108) (width 0.25) (layer B.Cu) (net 8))
 (segment (start 127.762 102.108) (end 127.762 86.360004) (width 0.25) (layer F.Cu) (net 8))
 (via (at 127.762 86.360004) (size 0.8) (drill 0.4) (layers F.Cu B.Cu) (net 8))
 (segment (start 127.761996 86.36) (end 127.762 86.360004) (width 0.25) (layer B.Cu) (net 8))
 (segment (start 117.094 86.36) (end 127.761996 86.36) (width 0.25) (layer B.Cu) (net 8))
 (segment (start 116.332 85.598) (end 117.094 86.36) (width 0.25) (layer B.Cu) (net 8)))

